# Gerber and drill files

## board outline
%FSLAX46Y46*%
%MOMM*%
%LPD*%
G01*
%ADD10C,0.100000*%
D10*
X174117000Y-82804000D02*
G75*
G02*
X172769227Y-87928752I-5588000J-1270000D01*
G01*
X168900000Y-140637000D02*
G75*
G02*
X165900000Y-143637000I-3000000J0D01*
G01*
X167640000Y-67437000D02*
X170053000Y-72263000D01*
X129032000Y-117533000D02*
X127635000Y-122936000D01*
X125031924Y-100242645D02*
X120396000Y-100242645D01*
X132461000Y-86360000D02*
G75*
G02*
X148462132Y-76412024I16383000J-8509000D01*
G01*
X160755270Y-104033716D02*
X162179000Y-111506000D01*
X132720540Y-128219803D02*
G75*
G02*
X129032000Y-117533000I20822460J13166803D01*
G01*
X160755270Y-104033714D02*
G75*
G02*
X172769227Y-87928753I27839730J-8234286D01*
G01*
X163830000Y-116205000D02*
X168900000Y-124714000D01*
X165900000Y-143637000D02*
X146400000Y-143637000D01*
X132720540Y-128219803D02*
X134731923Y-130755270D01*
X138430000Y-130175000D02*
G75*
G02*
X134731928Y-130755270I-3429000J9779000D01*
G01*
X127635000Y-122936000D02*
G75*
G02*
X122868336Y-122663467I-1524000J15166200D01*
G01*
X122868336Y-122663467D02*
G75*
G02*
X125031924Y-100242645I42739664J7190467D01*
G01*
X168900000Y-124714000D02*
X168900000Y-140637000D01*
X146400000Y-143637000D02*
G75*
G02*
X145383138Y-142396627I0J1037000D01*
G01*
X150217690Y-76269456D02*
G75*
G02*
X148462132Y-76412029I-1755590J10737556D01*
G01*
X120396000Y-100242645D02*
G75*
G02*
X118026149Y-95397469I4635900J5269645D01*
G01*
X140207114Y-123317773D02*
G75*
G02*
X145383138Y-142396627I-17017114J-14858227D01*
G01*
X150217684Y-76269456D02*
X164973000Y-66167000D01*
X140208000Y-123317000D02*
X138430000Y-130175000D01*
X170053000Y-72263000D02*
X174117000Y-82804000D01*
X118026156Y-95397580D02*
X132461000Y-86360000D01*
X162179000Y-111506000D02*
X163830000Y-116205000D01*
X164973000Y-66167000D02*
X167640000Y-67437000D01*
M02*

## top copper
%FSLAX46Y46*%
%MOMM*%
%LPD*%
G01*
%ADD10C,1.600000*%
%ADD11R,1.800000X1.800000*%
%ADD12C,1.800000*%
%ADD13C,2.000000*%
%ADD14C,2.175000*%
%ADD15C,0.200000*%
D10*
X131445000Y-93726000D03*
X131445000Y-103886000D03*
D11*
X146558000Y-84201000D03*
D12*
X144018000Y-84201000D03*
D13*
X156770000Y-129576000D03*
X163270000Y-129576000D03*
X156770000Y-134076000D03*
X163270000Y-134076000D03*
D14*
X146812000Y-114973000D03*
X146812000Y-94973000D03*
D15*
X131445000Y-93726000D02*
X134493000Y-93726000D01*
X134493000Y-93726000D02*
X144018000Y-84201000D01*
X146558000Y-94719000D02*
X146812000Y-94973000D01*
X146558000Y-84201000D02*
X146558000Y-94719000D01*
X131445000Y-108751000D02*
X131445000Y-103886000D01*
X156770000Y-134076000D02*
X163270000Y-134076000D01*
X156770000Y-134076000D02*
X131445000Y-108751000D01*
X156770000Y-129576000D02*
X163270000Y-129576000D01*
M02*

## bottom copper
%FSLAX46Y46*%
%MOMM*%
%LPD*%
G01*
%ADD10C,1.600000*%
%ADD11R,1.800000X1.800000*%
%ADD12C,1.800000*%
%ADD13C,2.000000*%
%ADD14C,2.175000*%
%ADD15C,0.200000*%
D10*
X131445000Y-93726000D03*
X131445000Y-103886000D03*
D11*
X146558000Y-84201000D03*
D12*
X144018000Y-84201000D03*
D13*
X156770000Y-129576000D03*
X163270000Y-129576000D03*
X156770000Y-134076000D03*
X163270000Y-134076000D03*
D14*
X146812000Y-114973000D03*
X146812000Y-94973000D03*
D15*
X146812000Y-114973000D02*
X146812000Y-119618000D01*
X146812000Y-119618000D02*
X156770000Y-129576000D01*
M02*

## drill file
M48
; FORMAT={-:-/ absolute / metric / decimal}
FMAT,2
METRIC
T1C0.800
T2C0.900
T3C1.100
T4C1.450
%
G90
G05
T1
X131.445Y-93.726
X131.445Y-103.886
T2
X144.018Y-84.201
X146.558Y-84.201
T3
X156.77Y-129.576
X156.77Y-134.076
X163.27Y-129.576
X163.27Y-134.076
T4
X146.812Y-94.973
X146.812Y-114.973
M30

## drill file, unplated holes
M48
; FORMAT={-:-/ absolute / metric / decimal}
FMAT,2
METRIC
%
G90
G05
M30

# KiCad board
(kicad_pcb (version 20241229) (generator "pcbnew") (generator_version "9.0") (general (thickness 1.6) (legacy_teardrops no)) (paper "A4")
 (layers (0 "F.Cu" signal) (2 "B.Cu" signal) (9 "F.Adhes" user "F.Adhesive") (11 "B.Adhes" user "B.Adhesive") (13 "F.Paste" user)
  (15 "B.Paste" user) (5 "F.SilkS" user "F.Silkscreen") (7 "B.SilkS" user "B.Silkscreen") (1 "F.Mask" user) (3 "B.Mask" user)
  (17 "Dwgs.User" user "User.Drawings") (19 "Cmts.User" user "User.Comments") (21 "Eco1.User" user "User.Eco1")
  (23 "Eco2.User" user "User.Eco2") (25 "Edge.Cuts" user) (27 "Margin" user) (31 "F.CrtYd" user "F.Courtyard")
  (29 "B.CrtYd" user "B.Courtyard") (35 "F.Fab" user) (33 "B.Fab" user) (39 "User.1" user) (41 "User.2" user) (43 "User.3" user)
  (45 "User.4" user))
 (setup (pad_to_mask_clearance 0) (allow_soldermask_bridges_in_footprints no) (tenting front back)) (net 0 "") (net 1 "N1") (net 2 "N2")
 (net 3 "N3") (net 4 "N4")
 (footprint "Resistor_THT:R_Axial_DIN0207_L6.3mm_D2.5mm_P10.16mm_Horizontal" (layer "F.Cu") (at 131.445 93.726 -90)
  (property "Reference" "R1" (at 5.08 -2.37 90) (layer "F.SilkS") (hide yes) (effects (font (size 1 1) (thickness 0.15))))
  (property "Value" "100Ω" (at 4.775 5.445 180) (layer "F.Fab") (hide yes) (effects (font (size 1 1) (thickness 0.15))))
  (pad "1" thru_hole circle (at 0 0 270) (size 1.6 1.6) (drill 0.8) (layers "*.Cu" "*.Mask") (remove_unused_layers no) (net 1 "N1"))
  (pad "2" thru_hole circle (at 10.16 0 270) (size 1.6 1.6) (drill 0.8) (layers "*.Cu" "*.Mask") (remove_unused_layers no) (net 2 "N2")))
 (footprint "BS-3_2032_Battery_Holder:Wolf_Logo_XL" (layer "F.Cu") (at 146.05 101.346)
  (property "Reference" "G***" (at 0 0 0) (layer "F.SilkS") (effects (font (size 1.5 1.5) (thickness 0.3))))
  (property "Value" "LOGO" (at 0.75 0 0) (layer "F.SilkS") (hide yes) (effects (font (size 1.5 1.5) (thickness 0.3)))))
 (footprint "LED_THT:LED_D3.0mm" (layer "F.Cu") (at 146.558 84.201 180)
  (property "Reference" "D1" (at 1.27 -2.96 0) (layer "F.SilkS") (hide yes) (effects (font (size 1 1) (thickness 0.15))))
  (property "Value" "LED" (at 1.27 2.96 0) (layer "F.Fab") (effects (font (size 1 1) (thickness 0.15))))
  (pad "1" thru_hole rect (at 0 0 180) (size 1.8 1.8) (drill 0.9) (layers "*.Cu" "*.Mask") (remove_unused_layers no) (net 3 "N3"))
  (pad "2" thru_hole circle (at 2.54 0 180) (size 1.8 1.8) (drill 0.9) (layers "*.Cu" "*.Mask") (remove_unused_layers no) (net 1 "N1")))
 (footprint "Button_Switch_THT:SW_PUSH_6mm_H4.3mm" (layer "F.Cu") (at 156.77 129.576)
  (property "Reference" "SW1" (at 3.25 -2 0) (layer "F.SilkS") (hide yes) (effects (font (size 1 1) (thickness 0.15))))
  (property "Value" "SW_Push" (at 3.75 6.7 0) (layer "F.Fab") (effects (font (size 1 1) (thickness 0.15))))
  (pad "1" thru_hole circle (at 0 0 90) (size 2 2) (drill 1.1) (layers "*.Cu" "*.Mask") (remove_unused_layers no) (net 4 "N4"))
  (pad "1" thru_hole circle (at 6.5 0 90) (size 2 2) (drill 1.1) (layers "*.Cu" "*.Mask") (remove_unused_layers no) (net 4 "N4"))
  (pad "2" thru_hole circle (at 0 4.5 90) (size 2 2) (drill 1.1) (layers "*.Cu" "*.Mask") (remove_unused_layers no) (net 2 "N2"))
  (pad "2" thru_hole circle (at 6.5 4.5 90) (size 2 2) (drill 1.1) (layers "*.Cu" "*.Mask") (remove_unused_layers no) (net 2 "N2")))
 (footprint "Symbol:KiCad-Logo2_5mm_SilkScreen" (layer "B.Cu") (at 151.13 123.063 180)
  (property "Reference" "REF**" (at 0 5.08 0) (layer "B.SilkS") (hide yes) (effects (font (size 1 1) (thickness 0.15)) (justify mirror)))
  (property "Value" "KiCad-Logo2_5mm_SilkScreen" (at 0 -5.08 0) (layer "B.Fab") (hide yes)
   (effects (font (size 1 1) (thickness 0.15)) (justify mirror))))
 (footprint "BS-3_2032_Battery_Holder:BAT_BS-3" (layer "B.Cu") (at 146.812 101.473 180)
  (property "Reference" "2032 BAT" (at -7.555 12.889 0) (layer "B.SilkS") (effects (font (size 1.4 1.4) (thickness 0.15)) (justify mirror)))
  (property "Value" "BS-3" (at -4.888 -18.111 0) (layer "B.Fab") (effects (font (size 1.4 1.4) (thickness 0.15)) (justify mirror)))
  (pad "+" thru_hole circle (at 0 -13.5 180) (size 2.175 2.175) (drill 1.45) (layers "*.Cu" "*.Mask") (remove_unused_layers no) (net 4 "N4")
   (solder_mask_margin 0.102))
  (pad "-" thru_hole circle (at 0 6.5 180) (size 2.175 2.175) (drill 1.45) (layers "*.Cu" "*.Mask") (remove_unused_layers no) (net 3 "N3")
   (solder_mask_margin 0.102)))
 (gr_arc (start 174.117 82.804) (mid 174.071047 85.531518) (end 172.769227 87.928752) (stroke (width 0.1) (type default))
  (layer "Edge.Cuts"))
 (gr_arc (start 168.9 140.637) (mid 168.02132 142.75832) (end 165.9 143.637) (stroke (width 0.1) (type default)) (layer "Edge.Cuts"))
 (gr_line (start 167.64 67.437) (end 170.053 72.263) (stroke (width 0.1) (type default)) (layer "Edge.Cuts"))
 (gr_line (start 129.032 117.533) (end 127.635 122.936) (stroke (width 0.1) (type default)) (layer "Edge.Cuts"))
 (gr_line (start 125.031924 100.242645) (end 120.396 100.242645) (stroke (width 0.1) (type default)) (layer "Edge.Cuts"))
 (gr_arc (start 132.461 86.36) (mid 139.09691 79.190989) (end 148.462132 76.412025) (stroke (width 0.1) (type default)) (layer "Edge.Cuts"))
 (gr_line (start 160.75527 104.033716) (end 162.179 111.506) (stroke (width 0.1) (type default)) (layer "Edge.Cuts"))
 (gr_arc (start 132.72054 128.219803) (mid 130.254964 123.090844) (end 129.032 117.533) (stroke (width 0.1) (type default))
  (layer "Edge.Cuts"))
 (gr_arc (start 160.75527 104.033714) (mid 165.324601 94.908779) (end 172.769227 87.928752) (stroke (width 0.1) (type default))
  (layer "Edge.Cuts"))
 (gr_line (start 163.83 116.205) (end 168.9 124.714) (stroke (width 0.1) (type default)) (layer "Edge.Cuts"))
 (gr_line (start 165.9 143.637) (end 146.4 143.637) (stroke (width 0.1) (type default)) (layer "Edge.Cuts"))
 (gr_line (start 132.72054 128.219803) (end 134.731923 130.75527) (stroke (width 0.1) (type default)) (layer "Edge.Cuts"))
 (gr_arc (start 138.43 130.175) (mid 136.607382 130.633501) (end 134.731928 130.75527) (stroke (width 0.1) (type default))
  (layer "Edge.Cuts"))
 (gr_arc (start 127.635 122.936) (mid 125.240931 122.987526) (end 122.868336 122.663467) (stroke (width 0.1) (type default))
  (layer "Edge.Cuts"))
 (gr_arc (start 122.868336 122.663467) (mid 122.468094 111.310041) (end 125.031924 100.242645) (stroke (width 0.1) (type default))
  (layer "Edge.Cuts"))
 (gr_line (start 168.9 124.714) (end 168.9 140.637) (stroke (width 0.1) (type default)) (layer "Edge.Cuts"))
 (gr_arc (start 146.4 143.637) (mid 145.598044 143.257446) (end 145.383138 142.396627) (stroke (width 0.1) (type solid)) (layer "Edge.Cuts"))
 (gr_arc (start 150.21769 76.269456) (mid 149.342801 76.376324) (end 148.462132 76.412025) (stroke (width 0.1) (type default))
  (layer "Edge.Cuts"))
 (gr_arc (start 120.396 100.242645) (mid 118.727071 98.056792) (end 118.026156 95.397469) (stroke (width 0.1) (type default))
  (layer "Edge.Cuts"))
 (gr_arc (start 140.207114 123.317773) (mid 144.99279 132.260982) (end 145.383138 142.396627) (stroke (width 0.1) (type default))
  (layer "Edge.Cuts"))
 (gr_line (start 150.217684 76.269456) (end 164.973 66.167) (stroke (width 0.1) (type default)) (layer "Edge.Cuts"))
 (gr_line (start 140.208 123.317) (end 138.43 130.175) (stroke (width 0.1) (type default)) (layer "Edge.Cuts"))
 (gr_line (start 170.053 72.263) (end 174.117 82.804) (stroke (width 0.1) (type default)) (layer "Edge.Cuts"))
 (gr_line (start 118.026156 95.39758) (end 132.461 86.36) (stroke (width 0.1) (type default)) (layer "Edge.Cuts"))
 (gr_line (start 162.179 111.506) (end 163.83 116.205) (stroke (width 0.1) (type default)) (layer "Edge.Cuts"))
 (gr_line (start 164.973 66.167) (end 167.64 67.437) (stroke (width 0.1) (type default)) (layer "Edge.Cuts"))
 (segment (start 131.445 93.726) (end 134.493 93.726) (width 0.2) (layer "F.Cu") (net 1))
 (segment (start 134.493 93.726) (end 144.018 84.201) (width 0.2) (layer "F.Cu") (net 1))
 (segment (start 146.558 94.719) (end 146.812 94.973) (width 0.2) (layer "F.Cu") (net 3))
 (segment (start 146.558 84.201) (end 146.558 94.719) (width 0.2) (layer "F.Cu") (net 3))
 (segment (start 131.445 108.751) (end 131.445 103.886) (width 0.2) (layer "F.Cu") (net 2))
 (segment (start 156.77 134.076) (end 163.27 134.076) (width 0.2) (layer "F.Cu") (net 2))
 (segment (start 156.77 134.076) (end 131.445 108.751) (width 0.2) (layer "F.Cu") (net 2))
 (segment (start 156.77 129.576) (end 163.27 129.576) (width 0.2) (layer "F.Cu") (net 4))
 (segment (start 146.812 114.973) (end 146.812 119.618) (width 0.2) (layer "B.Cu") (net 4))
 (segment (start 146.812 119.618) (end 156.77 129.576) (width 0.2) (layer "B.Cu") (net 4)))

